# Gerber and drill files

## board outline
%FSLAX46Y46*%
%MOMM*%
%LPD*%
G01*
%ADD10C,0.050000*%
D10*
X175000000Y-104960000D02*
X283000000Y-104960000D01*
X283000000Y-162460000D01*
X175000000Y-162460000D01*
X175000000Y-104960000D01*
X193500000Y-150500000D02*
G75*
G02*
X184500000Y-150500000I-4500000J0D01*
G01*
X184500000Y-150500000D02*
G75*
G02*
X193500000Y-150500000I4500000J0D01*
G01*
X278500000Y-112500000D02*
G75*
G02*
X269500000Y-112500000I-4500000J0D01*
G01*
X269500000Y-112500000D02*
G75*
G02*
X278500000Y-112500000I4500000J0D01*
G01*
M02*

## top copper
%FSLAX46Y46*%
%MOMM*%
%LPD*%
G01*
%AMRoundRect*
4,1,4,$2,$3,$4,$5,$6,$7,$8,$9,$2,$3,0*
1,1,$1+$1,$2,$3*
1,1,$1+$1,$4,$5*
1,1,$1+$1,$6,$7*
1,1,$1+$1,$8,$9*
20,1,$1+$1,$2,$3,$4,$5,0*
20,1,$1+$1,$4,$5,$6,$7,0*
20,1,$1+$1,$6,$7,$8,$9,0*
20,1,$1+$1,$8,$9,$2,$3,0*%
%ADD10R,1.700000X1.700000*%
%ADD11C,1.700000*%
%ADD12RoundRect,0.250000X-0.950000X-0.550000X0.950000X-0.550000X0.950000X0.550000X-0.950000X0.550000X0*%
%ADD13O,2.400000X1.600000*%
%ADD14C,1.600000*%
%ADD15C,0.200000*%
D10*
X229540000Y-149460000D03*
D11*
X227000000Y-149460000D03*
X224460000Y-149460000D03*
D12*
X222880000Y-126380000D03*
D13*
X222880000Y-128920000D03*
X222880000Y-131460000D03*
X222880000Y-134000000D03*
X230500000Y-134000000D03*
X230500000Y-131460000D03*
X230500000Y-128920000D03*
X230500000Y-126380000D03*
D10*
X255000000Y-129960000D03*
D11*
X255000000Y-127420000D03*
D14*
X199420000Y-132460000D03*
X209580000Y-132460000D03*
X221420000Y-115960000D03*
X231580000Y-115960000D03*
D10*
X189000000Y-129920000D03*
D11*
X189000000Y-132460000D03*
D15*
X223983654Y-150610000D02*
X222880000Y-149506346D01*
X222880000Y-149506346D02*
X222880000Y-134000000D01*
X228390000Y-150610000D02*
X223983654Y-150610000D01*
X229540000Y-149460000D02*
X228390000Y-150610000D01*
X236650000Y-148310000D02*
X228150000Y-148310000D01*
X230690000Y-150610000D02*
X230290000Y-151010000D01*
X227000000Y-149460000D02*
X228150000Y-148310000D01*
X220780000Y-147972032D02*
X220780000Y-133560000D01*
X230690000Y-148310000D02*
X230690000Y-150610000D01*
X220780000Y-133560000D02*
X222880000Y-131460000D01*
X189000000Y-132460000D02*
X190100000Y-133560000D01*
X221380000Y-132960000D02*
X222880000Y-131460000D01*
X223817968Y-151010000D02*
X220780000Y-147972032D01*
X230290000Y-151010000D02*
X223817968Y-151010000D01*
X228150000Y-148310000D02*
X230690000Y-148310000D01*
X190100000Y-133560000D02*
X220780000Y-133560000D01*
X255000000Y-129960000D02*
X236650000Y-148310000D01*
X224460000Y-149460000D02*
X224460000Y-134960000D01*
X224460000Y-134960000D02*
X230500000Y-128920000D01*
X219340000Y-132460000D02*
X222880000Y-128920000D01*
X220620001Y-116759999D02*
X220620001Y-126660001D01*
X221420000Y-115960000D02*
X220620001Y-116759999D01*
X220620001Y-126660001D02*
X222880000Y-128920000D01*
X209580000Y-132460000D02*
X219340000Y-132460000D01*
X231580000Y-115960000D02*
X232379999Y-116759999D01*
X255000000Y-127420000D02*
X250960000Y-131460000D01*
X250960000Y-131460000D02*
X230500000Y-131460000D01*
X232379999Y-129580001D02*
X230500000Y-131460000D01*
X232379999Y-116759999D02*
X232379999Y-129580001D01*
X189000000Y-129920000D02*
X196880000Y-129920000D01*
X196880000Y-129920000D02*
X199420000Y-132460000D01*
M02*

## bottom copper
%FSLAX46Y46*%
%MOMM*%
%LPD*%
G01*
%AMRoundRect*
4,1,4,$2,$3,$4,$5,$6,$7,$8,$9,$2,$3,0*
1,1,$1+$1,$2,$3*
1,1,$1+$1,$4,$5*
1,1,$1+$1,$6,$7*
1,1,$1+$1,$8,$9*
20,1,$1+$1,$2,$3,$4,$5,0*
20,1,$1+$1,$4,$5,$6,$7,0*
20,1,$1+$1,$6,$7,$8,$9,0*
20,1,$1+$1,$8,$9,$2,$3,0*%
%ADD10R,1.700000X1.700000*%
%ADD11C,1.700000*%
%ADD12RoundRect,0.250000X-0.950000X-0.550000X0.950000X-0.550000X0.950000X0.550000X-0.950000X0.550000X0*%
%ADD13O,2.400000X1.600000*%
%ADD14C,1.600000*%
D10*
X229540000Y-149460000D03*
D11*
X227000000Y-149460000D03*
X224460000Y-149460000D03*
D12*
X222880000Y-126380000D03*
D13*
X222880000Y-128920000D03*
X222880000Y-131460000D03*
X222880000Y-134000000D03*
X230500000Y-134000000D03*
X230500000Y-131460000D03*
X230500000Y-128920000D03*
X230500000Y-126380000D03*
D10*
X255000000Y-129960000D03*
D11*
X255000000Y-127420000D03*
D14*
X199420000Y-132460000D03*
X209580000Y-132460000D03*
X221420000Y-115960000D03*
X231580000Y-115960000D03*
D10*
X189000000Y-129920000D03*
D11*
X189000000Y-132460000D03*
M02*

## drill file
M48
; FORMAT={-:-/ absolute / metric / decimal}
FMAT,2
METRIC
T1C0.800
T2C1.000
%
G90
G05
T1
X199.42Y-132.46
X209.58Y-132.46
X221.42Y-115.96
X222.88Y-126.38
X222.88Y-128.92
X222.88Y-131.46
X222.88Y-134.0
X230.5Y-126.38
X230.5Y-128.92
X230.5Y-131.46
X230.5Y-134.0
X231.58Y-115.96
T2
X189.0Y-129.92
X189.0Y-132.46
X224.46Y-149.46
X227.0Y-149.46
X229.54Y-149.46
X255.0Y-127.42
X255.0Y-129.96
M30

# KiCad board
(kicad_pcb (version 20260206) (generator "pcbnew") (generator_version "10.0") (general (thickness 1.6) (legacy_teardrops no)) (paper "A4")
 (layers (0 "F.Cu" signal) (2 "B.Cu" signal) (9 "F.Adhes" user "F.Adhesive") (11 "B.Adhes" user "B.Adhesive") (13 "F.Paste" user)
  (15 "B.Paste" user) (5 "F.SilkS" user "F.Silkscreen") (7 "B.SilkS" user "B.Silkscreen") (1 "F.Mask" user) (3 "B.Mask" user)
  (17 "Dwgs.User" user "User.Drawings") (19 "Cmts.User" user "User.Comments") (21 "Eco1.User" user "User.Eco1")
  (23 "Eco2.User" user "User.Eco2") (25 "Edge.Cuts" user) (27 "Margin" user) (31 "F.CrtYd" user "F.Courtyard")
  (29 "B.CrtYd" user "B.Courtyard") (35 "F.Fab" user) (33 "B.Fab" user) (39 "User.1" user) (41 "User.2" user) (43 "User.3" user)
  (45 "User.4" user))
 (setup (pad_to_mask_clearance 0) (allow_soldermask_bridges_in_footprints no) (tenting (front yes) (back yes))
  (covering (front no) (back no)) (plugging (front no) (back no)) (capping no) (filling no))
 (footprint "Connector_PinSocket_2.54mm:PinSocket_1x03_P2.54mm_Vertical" (layer "F.Cu") (at 229.54 149.46 -90)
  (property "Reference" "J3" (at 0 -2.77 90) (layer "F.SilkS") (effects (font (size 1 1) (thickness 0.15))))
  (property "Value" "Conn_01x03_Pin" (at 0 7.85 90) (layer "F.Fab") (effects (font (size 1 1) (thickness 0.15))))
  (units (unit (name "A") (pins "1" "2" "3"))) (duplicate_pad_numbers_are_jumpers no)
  (pad "1" thru_hole rect (at 0 0 270) (size 1.7 1.7) (drill 1) (layers "*.Cu" "*.Mask") (remove_unused_layers no) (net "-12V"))
  (pad "2" thru_hole circle (at 0 2.54 270) (size 1.7 1.7) (drill 1) (layers "*.Cu" "*.Mask") (remove_unused_layers no) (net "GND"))
  (pad "3" thru_hole circle (at 0 5.08 270) (size 1.7 1.7) (drill 1) (layers "*.Cu" "*.Mask") (remove_unused_layers no) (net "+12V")))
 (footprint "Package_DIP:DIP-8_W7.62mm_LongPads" (layer "F.Cu") (at 222.88 126.38)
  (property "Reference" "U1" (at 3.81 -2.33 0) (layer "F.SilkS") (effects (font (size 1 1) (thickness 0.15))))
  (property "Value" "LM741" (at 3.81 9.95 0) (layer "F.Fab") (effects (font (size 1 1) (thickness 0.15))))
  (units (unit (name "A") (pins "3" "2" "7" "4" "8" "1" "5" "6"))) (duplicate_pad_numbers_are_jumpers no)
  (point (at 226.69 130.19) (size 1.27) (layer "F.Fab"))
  (pad "1" thru_hole roundrect (at 0 0) (size 2.4 1.6) (drill 0.8) (layers "*.Cu" "*.Mask") (remove_unused_layers no)
   (roundrect_rratio 0.15625) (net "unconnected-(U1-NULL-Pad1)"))
  (pad "2" thru_hole oval (at 0 2.54) (size 2.4 1.6) (drill 0.8) (layers "*.Cu" "*.Mask") (remove_unused_layers no) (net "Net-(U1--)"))
  (pad "3" thru_hole oval (at 0 5.08) (size 2.4 1.6) (drill 0.8) (layers "*.Cu" "*.Mask") (remove_unused_layers no) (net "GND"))
  (pad "4" thru_hole oval (at 0 7.62) (size 2.4 1.6) (drill 0.8) (layers "*.Cu" "*.Mask") (remove_unused_layers no) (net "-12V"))
  (pad "5" thru_hole oval (at 7.62 7.62) (size 2.4 1.6) (drill 0.8) (layers "*.Cu" "*.Mask") (remove_unused_layers no)
   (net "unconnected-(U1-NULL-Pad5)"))
  (pad "6" thru_hole oval (at 7.62 5.08) (size 2.4 1.6) (drill 0.8) (layers "*.Cu" "*.Mask") (remove_unused_layers no)
   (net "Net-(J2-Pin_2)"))
  (pad "7" thru_hole oval (at 7.62 2.54) (size 2.4 1.6) (drill 0.8) (layers "*.Cu" "*.Mask") (remove_unused_layers no) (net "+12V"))
  (pad "8" thru_hole oval (at 7.62 0) (size 2.4 1.6) (drill 0.8) (layers "*.Cu" "*.Mask") (remove_unused_layers no)
   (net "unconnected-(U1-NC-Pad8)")))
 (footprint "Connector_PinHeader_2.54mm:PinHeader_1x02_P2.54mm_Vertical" (layer "F.Cu") (at 255 129.96 180)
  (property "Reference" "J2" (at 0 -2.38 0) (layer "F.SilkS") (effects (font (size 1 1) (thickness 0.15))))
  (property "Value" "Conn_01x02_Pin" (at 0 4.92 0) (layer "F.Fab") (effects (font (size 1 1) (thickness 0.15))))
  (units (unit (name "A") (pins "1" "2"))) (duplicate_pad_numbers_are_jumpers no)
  (pad "1" thru_hole rect (at 0 0 180) (size 1.7 1.7) (drill 1) (layers "*.Cu" "*.Mask") (remove_unused_layers no) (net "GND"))
  (pad "2" thru_hole circle (at 0 2.54 180) (size 1.7 1.7) (drill 1) (layers "*.Cu" "*.Mask") (remove_unused_layers no)
   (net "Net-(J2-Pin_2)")))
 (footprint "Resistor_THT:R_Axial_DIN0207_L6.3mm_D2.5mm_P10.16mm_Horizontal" (layer "F.Cu") (at 199.42 132.46)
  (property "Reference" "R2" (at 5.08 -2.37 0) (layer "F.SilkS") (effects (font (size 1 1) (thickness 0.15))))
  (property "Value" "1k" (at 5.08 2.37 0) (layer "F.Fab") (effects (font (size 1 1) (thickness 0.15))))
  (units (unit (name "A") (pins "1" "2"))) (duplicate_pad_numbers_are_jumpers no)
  (pad "1" thru_hole circle (at 0 0) (size 1.6 1.6) (drill 0.8) (layers "*.Cu" "*.Mask") (remove_unused_layers no) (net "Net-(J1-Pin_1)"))
  (pad "2" thru_hole circle (at 10.16 0) (size 1.6 1.6) (drill 0.8) (layers "*.Cu" "*.Mask") (remove_unused_layers no) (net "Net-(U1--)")))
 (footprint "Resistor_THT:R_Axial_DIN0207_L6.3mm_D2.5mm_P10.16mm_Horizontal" (layer "F.Cu") (at 221.42 115.96)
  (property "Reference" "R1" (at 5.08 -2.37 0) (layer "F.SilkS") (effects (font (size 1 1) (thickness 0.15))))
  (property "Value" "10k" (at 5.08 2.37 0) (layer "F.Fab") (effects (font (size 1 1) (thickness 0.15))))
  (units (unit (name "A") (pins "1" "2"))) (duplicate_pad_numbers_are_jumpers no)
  (pad "1" thru_hole circle (at 0 0) (size 1.6 1.6) (drill 0.8) (layers "*.Cu" "*.Mask") (remove_unused_layers no) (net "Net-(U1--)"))
  (pad "2" thru_hole circle (at 10.16 0) (size 1.6 1.6) (drill 0.8) (layers "*.Cu" "*.Mask") (remove_unused_layers no)
   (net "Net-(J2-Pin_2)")))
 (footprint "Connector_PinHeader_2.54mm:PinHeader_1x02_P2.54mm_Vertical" (layer "F.Cu") (at 189 129.92)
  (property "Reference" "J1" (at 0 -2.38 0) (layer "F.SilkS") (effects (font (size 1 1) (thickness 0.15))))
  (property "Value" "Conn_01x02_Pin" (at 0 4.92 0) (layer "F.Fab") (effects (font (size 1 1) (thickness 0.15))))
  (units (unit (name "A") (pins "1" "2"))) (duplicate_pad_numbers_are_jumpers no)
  (pad "1" thru_hole rect (at 0 0) (size 1.7 1.7) (drill 1) (layers "*.Cu" "*.Mask") (remove_unused_layers no) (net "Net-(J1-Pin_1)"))
  (pad "2" thru_hole circle (at 0 2.54) (size 1.7 1.7) (drill 1) (layers "*.Cu" "*.Mask") (remove_unused_layers no) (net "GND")))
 (gr_rect (start 175 104.96) (end 283 162.46) (stroke (width 0.05) (type default)) (fill no) (layer "Edge.Cuts"))
 (gr_circle (center 189 150.5) (end 193.5 150.5) (stroke (width 0.05) (type solid)) (fill no) (layer "Edge.Cuts"))
 (gr_circle (center 274 112.5) (end 278.5 112.5) (stroke (width 0.05) (type solid)) (fill no) (layer "Edge.Cuts"))
 (segment (start 223.983654 150.61) (end 222.88 149.506346) (width 0.2) (layer "F.Cu") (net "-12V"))
 (segment (start 222.88 149.506346) (end 222.88 134) (width 0.2) (layer "F.Cu") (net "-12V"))
 (segment (start 228.39 150.61) (end 223.983654 150.61) (width 0.2) (layer "F.Cu") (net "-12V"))
 (segment (start 229.54 149.46) (end 228.39 150.61) (width 0.2) (layer "F.Cu") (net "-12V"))
 (segment (start 236.65 148.31) (end 228.15 148.31) (width 0.2) (layer "F.Cu") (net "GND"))
 (segment (start 230.69 150.61) (end 230.29 151.01) (width 0.2) (layer "F.Cu") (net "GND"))
 (segment (start 227 149.46) (end 228.15 148.31) (width 0.2) (layer "F.Cu") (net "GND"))
 (segment (start 220.78 147.972032) (end 220.78 133.56) (width 0.2) (layer "F.Cu") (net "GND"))
 (segment (start 230.69 148.31) (end 230.69 150.61) (width 0.2) (layer "F.Cu") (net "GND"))
 (segment (start 220.78 133.56) (end 222.88 131.46) (width 0.2) (layer "F.Cu") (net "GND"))
 (segment (start 189 132.46) (end 190.1 133.56) (width 0.2) (layer "F.Cu") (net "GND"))
 (segment (start 221.38 132.96) (end 222.88 131.46) (width 0.2) (layer "F.Cu") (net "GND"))
 (segment (start 223.817968 151.01) (end 220.78 147.972032) (width 0.2) (layer "F.Cu") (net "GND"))
 (segment (start 230.29 151.01) (end 223.817968 151.01) (width 0.2) (layer "F.Cu") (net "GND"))
 (segment (start 228.15 148.31) (end 230.69 148.31) (width 0.2) (layer "F.Cu") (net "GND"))
 (segment (start 190.1 133.56) (end 220.78 133.56) (width 0.2) (layer "F.Cu") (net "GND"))
 (segment (start 255 129.96) (end 236.65 148.31) (width 0.2) (layer "F.Cu") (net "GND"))
 (segment (start 224.46 149.46) (end 224.46 134.96) (width 0.2) (layer "F.Cu") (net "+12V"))
 (segment (start 224.46 134.96) (end 230.5 128.92) (width 0.2) (layer "F.Cu") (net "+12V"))
 (segment (start 219.34 132.46) (end 222.88 128.92) (width 0.2) (layer "F.Cu") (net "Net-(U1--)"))
 (segment (start 220.620001 116.759999) (end 220.620001 126.660001) (width 0.2) (layer "F.Cu") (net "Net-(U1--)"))
 (segment (start 221.42 115.96) (end 220.620001 116.759999) (width 0.2) (layer "F.Cu") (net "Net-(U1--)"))
 (segment (start 220.620001 126.660001) (end 222.88 128.92) (width 0.2) (layer "F.Cu") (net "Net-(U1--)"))
 (segment (start 209.58 132.46) (end 219.34 132.46) (width 0.2) (layer "F.Cu") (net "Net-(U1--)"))
 (segment (start 231.58 115.96) (end 232.379999 116.759999) (width 0.2) (layer "F.Cu") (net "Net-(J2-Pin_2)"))
 (segment (start 255 127.42) (end 250.96 131.46) (width 0.2) (layer "F.Cu") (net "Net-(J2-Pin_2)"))
 (segment (start 250.96 131.46) (end 230.5 131.46) (width 0.2) (layer "F.Cu") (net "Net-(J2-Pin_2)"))
 (segment (start 232.379999 129.580001) (end 230.5 131.46) (width 0.2) (layer "F.Cu") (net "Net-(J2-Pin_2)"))
 (segment (start 232.379999 116.759999) (end 232.379999 129.580001) (width 0.2) (layer "F.Cu") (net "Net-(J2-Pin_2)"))
 (segment (start 189 129.92) (end 196.88 129.92) (width 0.2) (layer "F.Cu") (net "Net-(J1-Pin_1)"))
 (segment (start 196.88 129.92) (end 199.42 132.46) (width 0.2) (layer "F.Cu") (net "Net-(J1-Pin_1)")))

